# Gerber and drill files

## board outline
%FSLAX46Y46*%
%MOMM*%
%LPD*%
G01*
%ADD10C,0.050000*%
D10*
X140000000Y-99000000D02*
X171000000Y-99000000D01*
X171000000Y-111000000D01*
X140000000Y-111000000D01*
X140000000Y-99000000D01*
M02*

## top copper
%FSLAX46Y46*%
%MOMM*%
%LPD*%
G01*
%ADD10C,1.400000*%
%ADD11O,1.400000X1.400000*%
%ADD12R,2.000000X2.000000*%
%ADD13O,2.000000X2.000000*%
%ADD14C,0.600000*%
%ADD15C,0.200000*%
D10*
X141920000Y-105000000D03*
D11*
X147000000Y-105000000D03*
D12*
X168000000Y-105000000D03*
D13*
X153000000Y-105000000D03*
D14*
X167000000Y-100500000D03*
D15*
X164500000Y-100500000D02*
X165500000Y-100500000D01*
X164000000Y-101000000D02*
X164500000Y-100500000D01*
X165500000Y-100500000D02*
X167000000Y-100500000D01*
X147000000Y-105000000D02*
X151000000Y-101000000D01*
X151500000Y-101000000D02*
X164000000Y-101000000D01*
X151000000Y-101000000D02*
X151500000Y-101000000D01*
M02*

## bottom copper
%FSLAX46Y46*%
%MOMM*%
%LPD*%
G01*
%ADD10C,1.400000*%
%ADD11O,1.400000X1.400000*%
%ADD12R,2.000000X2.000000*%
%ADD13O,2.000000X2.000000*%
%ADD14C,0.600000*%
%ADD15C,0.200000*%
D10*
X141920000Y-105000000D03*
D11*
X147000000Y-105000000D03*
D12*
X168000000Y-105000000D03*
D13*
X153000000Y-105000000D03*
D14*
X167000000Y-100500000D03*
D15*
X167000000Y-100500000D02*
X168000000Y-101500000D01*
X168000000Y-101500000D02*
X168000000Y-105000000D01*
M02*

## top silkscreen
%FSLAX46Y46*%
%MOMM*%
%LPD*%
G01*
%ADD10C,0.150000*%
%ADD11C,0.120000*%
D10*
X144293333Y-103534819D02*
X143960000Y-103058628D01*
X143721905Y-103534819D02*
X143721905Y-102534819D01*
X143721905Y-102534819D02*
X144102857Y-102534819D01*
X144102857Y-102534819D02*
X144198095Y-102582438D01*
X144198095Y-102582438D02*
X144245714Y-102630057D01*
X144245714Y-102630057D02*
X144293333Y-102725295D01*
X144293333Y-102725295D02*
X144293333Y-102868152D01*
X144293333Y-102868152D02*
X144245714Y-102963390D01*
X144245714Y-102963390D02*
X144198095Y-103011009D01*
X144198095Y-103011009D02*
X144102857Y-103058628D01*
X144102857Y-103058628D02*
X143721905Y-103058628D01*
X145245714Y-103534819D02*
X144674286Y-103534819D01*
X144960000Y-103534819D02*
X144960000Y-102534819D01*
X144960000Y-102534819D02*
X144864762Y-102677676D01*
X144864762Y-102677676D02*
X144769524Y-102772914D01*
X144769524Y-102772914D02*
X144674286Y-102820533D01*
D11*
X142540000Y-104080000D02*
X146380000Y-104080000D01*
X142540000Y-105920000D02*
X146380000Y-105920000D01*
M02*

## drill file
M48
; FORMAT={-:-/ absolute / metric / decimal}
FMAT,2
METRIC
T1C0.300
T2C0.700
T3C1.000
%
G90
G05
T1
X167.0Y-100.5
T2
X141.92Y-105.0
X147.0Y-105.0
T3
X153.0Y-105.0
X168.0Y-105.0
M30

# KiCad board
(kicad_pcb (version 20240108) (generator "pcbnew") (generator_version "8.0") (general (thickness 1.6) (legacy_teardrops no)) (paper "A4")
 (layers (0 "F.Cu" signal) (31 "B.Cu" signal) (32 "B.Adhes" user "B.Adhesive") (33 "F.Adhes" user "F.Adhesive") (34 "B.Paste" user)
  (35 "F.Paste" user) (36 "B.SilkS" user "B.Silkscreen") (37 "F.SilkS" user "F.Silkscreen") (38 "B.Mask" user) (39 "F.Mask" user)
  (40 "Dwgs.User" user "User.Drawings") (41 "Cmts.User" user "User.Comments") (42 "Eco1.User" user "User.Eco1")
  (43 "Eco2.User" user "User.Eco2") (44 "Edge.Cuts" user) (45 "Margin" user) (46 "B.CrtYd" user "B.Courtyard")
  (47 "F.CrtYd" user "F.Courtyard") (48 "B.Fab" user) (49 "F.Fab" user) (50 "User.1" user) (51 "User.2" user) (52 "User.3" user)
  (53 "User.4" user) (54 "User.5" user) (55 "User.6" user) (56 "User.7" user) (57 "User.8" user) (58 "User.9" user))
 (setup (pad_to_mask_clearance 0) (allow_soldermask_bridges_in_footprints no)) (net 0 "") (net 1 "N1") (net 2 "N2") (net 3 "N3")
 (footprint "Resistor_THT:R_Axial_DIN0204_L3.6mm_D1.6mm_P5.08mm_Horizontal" (layer "F.Cu") (at 141.92 105)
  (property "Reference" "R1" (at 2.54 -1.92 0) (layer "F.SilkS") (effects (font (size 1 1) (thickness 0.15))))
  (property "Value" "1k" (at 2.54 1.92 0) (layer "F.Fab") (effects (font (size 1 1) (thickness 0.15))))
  (fp_line (start 0.62 -0.92) (end 4.46 -0.92) (stroke (width 0.12) (type solid)) (layer "F.SilkS"))
  (fp_line (start 0.62 0.92) (end 4.46 0.92) (stroke (width 0.12) (type solid)) (layer "F.SilkS"))
  (pad "1" thru_hole circle (at 0 0) (size 1.4 1.4) (drill 0.7) (layers "*.Cu" "*.Mask") (remove_unused_layers no) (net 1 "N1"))
  (pad "2" thru_hole oval (at 5.08 0) (size 1.4 1.4) (drill 0.7) (layers "*.Cu" "*.Mask") (remove_unused_layers no) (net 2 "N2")))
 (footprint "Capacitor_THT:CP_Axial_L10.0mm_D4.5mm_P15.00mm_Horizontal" (layer "B.Cu") (at 168 105 180)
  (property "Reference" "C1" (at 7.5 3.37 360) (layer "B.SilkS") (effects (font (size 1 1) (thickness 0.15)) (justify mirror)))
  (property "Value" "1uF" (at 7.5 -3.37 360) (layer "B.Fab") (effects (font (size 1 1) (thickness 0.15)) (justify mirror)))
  (pad "1" thru_hole rect (at 0 0 180) (size 2 2) (drill 1) (layers "*.Cu" "*.Mask") (remove_unused_layers no) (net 2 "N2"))
  (pad "2" thru_hole oval (at 15 0 180) (size 2 2) (drill 1) (layers "*.Cu" "*.Mask") (remove_unused_layers no) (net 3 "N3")))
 (gr_rect (start 140 99) (end 171 111) (stroke (width 0.05) (type default)) (fill none) (layer "Edge.Cuts"))
 (segment (start 164.5 100.5) (end 165.5 100.5) (width 0.2) (layer "F.Cu") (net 2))
 (segment (start 164 101) (end 164.5 100.5) (width 0.2) (layer "F.Cu") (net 2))
 (segment (start 165.5 100.5) (end 167 100.5) (width 0.2) (layer "F.Cu") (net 2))
 (segment (start 147 105) (end 151 101) (width 0.2) (layer "F.Cu") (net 2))
 (segment (start 151.5 101) (end 164 101) (width 0.2) (layer "F.Cu") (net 2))
 (segment (start 151 101) (end 151.5 101) (width 0.2) (layer "F.Cu") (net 2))
 (via (at 167 100.5) (size 0.6) (drill 0.3) (layers "F.Cu" "B.Cu") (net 2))
 (segment (start 167 100.5) (end 168 101.5) (width 0.2) (layer "B.Cu") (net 2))
 (segment (start 168 101.5) (end 168 105) (width 0.2) (layer "B.Cu") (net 2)))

